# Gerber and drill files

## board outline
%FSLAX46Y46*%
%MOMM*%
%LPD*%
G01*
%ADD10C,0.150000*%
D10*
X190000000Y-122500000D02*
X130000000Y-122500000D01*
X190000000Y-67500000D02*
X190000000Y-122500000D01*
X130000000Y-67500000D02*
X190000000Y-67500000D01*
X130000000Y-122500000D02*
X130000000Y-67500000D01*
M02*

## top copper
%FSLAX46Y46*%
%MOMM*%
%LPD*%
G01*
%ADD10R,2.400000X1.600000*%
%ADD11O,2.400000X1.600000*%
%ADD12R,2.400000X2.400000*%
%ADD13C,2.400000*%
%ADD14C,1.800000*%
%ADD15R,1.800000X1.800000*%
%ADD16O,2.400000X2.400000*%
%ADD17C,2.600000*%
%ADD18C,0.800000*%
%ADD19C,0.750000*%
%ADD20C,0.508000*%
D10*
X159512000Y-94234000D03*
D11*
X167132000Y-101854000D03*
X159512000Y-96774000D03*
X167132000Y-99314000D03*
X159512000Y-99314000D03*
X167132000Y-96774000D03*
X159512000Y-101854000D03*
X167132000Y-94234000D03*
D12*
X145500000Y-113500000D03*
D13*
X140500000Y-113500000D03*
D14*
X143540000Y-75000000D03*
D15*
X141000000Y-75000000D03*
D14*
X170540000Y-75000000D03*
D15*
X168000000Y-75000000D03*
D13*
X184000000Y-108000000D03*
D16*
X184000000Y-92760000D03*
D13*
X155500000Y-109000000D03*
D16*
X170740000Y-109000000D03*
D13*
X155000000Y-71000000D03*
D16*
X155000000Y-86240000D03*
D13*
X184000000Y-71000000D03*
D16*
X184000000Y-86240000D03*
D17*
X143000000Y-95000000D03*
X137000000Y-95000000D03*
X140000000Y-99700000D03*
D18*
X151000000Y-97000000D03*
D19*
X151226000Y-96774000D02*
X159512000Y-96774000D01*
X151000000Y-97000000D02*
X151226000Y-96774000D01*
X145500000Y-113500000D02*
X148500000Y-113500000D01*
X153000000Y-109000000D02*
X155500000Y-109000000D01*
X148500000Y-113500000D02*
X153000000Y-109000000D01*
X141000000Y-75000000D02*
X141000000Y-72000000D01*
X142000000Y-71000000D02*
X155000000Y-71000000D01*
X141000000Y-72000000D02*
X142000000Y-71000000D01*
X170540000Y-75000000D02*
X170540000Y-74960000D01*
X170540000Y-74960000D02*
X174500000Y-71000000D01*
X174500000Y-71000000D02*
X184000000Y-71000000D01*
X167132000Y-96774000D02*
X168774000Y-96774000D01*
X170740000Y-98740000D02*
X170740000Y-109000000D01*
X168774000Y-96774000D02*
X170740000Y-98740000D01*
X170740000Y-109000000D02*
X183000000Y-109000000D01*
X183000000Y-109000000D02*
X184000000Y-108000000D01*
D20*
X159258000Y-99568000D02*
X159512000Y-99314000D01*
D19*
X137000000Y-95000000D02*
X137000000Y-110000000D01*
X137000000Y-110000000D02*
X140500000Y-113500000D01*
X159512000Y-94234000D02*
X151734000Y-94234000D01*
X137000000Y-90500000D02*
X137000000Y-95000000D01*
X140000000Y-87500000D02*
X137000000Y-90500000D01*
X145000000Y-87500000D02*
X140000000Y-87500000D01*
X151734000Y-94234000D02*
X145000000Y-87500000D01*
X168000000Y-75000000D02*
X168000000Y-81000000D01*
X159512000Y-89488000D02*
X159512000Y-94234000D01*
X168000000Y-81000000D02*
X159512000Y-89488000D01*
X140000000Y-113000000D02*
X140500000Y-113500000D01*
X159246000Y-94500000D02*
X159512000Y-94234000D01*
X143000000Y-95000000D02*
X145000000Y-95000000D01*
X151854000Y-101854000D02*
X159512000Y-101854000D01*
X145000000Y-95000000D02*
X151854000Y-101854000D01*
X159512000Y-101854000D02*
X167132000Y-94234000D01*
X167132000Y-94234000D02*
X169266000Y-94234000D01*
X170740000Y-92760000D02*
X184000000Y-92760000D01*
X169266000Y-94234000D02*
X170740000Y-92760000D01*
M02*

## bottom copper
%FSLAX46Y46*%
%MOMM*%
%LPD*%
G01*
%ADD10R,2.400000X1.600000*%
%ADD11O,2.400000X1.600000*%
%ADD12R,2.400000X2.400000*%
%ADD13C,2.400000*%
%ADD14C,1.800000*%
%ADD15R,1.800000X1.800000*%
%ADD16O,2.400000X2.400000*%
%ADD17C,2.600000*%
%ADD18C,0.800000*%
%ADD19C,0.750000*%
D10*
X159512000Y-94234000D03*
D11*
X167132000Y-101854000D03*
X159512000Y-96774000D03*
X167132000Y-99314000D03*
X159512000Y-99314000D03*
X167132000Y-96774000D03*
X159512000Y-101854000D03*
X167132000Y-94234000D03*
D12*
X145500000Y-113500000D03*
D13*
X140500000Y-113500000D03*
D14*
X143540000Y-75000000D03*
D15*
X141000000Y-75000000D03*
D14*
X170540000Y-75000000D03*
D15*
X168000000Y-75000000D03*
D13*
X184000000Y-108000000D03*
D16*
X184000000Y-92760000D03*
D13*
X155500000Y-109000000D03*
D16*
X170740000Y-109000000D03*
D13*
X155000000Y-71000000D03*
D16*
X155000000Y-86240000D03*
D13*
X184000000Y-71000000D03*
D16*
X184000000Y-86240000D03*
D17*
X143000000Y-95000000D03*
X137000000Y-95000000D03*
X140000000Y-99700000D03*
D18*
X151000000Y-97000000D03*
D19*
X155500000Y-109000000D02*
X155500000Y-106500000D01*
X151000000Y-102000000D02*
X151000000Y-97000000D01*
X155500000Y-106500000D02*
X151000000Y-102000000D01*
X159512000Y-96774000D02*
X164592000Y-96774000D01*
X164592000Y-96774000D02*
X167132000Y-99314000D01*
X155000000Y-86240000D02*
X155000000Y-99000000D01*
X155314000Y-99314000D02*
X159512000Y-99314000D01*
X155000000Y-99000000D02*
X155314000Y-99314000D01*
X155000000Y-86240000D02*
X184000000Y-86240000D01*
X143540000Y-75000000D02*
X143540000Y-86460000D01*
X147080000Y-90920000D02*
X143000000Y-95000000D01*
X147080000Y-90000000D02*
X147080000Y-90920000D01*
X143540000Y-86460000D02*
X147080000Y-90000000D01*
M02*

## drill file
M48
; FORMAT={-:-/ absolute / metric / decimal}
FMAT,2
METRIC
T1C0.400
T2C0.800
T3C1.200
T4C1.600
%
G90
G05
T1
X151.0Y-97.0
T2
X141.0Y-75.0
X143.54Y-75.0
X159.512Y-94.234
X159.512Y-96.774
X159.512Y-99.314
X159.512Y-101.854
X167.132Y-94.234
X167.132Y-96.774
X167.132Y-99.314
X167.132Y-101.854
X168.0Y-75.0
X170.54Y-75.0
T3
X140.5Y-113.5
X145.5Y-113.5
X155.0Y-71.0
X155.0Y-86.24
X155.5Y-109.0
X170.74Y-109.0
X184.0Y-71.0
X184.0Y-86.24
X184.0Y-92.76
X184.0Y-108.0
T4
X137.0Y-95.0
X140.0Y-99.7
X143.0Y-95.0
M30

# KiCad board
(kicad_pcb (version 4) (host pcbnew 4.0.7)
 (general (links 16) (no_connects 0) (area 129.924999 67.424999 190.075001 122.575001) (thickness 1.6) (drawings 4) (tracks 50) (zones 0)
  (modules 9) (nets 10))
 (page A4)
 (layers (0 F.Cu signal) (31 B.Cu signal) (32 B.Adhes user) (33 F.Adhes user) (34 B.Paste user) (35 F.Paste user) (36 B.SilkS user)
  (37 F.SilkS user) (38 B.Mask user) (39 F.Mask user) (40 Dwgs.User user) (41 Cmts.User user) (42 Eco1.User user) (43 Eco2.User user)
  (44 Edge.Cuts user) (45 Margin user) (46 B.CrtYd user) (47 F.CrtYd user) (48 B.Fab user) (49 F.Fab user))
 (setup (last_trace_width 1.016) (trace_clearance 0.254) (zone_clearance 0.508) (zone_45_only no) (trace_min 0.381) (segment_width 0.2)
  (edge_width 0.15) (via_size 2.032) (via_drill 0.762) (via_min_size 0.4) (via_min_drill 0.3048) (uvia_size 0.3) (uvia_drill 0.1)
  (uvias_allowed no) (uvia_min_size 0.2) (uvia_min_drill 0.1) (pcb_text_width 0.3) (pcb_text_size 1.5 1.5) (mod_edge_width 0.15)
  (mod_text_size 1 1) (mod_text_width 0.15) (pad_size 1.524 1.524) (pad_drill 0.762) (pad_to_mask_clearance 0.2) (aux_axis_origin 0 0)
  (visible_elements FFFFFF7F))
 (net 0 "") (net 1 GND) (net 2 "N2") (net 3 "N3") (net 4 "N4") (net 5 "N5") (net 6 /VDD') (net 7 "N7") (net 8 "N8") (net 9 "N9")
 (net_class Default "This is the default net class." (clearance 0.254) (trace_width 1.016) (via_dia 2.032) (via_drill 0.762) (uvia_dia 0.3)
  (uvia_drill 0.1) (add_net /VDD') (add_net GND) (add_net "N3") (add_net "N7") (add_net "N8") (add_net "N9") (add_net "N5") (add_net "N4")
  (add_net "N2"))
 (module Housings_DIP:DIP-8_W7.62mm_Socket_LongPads (layer F.Cu) (at 159.512 94.234)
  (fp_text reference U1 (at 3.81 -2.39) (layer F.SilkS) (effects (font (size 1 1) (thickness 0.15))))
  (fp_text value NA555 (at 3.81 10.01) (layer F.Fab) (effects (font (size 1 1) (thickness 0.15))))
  (pad 1 thru_hole rect (at 0 0) (size 2.4 1.6) (drill 0.8) (layers *.Cu *.Mask) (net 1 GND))
  (pad 5 thru_hole oval (at 7.62 7.62) (size 2.4 1.6) (drill 0.8) (layers *.Cu *.Mask) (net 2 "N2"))
  (pad 2 thru_hole oval (at 0 2.54) (size 2.4 1.6) (drill 0.8) (layers *.Cu *.Mask) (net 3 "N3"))
  (pad 6 thru_hole oval (at 7.62 5.08) (size 2.4 1.6) (drill 0.8) (layers *.Cu *.Mask) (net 3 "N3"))
  (pad 3 thru_hole oval (at 0 5.08) (size 2.4 1.6) (drill 0.8) (layers *.Cu *.Mask) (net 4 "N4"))
  (pad 7 thru_hole oval (at 7.62 2.54) (size 2.4 1.6) (drill 0.8) (layers *.Cu *.Mask) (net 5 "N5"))
  (pad 4 thru_hole oval (at 0 7.62) (size 2.4 1.6) (drill 0.8) (layers *.Cu *.Mask) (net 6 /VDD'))
  (pad 8 thru_hole oval (at 7.62 0) (size 2.4 1.6) (drill 0.8) (layers *.Cu *.Mask) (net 6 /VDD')))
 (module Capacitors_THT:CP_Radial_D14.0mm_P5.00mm (layer F.Cu) (at 145.5 113.5 180)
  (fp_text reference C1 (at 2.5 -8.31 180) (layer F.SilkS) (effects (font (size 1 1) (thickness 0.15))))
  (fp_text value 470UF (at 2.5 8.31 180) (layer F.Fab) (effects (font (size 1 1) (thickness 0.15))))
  (pad 1 thru_hole rect (at 0 0 180) (size 2.4 2.4) (drill 1.2) (layers *.Cu *.Mask) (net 3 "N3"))
  (pad 2 thru_hole circle (at 5 0 180) (size 2.4 2.4) (drill 1.2) (layers *.Cu *.Mask) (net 1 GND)))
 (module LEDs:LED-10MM (layer F.Cu) (at 141 75)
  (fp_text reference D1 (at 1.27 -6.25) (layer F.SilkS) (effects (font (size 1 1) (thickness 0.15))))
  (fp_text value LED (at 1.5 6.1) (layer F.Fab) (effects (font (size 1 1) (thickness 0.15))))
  (pad 2 thru_hole circle (at 2.54 0 180) (size 1.8 1.8) (drill 0.8) (layers *.Cu *.Mask) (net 6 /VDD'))
  (pad 1 thru_hole rect (at 0 0 180) (size 1.8 1.8) (drill 0.8) (layers *.Cu *.Mask) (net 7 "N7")))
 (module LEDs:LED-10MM (layer F.Cu) (at 168 75)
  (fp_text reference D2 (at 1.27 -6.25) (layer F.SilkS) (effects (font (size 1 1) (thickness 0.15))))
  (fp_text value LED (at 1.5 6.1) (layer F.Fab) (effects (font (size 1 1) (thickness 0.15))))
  (pad 2 thru_hole circle (at 2.54 0 180) (size 1.8 1.8) (drill 0.8) (layers *.Cu *.Mask) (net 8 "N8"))
  (pad 1 thru_hole rect (at 0 0 180) (size 1.8 1.8) (drill 0.8) (layers *.Cu *.Mask) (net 1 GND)))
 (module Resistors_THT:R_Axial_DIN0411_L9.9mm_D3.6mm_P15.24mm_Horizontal (layer F.Cu) (at 184 108 90)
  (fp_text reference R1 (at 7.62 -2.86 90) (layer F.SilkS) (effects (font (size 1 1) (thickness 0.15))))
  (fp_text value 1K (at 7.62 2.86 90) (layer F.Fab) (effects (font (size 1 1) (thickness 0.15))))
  (pad 1 thru_hole circle (at 0 0 90) (size 2.4 2.4) (drill 1.2) (layers *.Cu *.Mask) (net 5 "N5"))
  (pad 2 thru_hole oval (at 15.24 0 90) (size 2.4 2.4) (drill 1.2) (layers *.Cu *.Mask) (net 6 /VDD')))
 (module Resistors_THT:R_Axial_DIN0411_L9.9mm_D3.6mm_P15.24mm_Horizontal (layer F.Cu) (at 155.5 109)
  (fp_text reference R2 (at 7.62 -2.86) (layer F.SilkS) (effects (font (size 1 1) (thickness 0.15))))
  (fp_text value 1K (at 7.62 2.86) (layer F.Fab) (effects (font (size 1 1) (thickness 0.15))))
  (pad 1 thru_hole circle (at 0 0) (size 2.4 2.4) (drill 1.2) (layers *.Cu *.Mask) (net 3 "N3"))
  (pad 2 thru_hole oval (at 15.24 0) (size 2.4 2.4) (drill 1.2) (layers *.Cu *.Mask) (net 5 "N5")))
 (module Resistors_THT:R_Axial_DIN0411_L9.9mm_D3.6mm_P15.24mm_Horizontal (layer F.Cu) (at 155 71 270)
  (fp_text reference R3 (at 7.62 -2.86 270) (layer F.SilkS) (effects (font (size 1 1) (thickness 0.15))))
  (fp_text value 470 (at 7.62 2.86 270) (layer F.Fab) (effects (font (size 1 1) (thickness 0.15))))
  (pad 1 thru_hole circle (at 0 0 270) (size 2.4 2.4) (drill 1.2) (layers *.Cu *.Mask) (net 7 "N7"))
  (pad 2 thru_hole oval (at 15.24 0 270) (size 2.4 2.4) (drill 1.2) (layers *.Cu *.Mask) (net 4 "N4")))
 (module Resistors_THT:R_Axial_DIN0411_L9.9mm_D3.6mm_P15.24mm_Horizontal (layer F.Cu) (at 184 71 270)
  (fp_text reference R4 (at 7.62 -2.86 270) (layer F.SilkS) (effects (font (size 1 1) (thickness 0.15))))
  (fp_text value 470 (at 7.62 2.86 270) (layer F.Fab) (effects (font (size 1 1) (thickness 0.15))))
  (pad 1 thru_hole circle (at 0 0 270) (size 2.4 2.4) (drill 1.2) (layers *.Cu *.Mask) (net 8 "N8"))
  (pad 2 thru_hole oval (at 15.24 0 270) (size 2.4 2.4) (drill 1.2) (layers *.Cu *.Mask) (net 4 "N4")))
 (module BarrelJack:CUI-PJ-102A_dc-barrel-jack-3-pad (layer F.Cu) (at 140 95 90)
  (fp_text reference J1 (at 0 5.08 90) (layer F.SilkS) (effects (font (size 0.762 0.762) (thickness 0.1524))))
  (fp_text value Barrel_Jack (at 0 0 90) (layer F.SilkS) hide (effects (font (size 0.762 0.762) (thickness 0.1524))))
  (pad 1 thru_hole circle (at 0 3 90) (size 2.6 2.6) (drill 1.6) (layers *.Cu *.Mask F.SilkS) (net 6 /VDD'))
  (pad 2 thru_hole circle (at 0 -3 90) (size 2.6 2.6) (drill 1.6) (layers *.Cu *.Mask F.SilkS) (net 1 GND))
  (pad 3 thru_hole circle (at -4.7 0 90) (size 2.6 2.6) (drill 1.6) (layers *.Cu *.Mask F.SilkS) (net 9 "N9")))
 (gr_line (start 190 122.5) (end 130 122.5) (angle 90) (layer Edge.Cuts) (width 0.15))
 (gr_line (start 190 67.5) (end 190 122.5) (angle 90) (layer Edge.Cuts) (width 0.15))
 (gr_line (start 130 67.5) (end 190 67.5) (angle 90) (layer Edge.Cuts) (width 0.15))
 (gr_line (start 130 122.5) (end 130 67.5) (angle 90) (layer Edge.Cuts) (width 0.15))
 (segment (start 155.5 109) (end 155.5 106.5) (width 0.75) (layer B.Cu) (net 3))
 (segment (start 151.226 96.774) (end 159.512 96.774) (width 0.75) (layer F.Cu) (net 3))
 (segment (start 151 97) (end 151.226 96.774) (width 0.75) (layer F.Cu) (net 3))
 (via (at 151 97) (size 0.8) (drill 0.4) (layers F.Cu B.Cu) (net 3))
 (segment (start 151 102) (end 151 97) (width 0.75) (layer B.Cu) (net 3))
 (segment (start 155.5 106.5) (end 151 102) (width 0.75) (layer B.Cu) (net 3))
 (segment (start 159.512 96.774) (end 164.592 96.774) (width 0.75) (layer B.Cu) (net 3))
 (segment (start 164.592 96.774) (end 167.132 99.314) (width 0.75) (layer B.Cu) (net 3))
 (segment (start 145.5 113.5) (end 148.5 113.5) (width 0.75) (layer F.Cu) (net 3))
 (segment (start 153 109) (end 155.5 109) (width 0.75) (layer F.Cu) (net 3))
 (segment (start 148.5 113.5) (end 153 109) (width 0.75) (layer F.Cu) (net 3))
 (segment (start 141 75) (end 141 72) (width 0.75) (layer F.Cu) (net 7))
 (segment (start 142 71) (end 155 71) (width 0.75) (layer F.Cu) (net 7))
 (segment (start 141 72) (end 142 71) (width 0.75) (layer F.Cu) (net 7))
 (segment (start 170.54 75) (end 170.54 74.96) (width 0.75) (layer F.Cu) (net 8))
 (segment (start 170.54 74.96) (end 174.5 71) (width 0.75) (layer F.Cu) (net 8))
 (segment (start 174.5 71) (end 184 71) (width 0.75) (layer F.Cu) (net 8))
 (segment (start 167.132 96.774) (end 168.774 96.774) (width 0.75) (layer F.Cu) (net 5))
 (segment (start 170.74 98.74) (end 170.74 109) (width 0.75) (layer F.Cu) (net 5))
 (segment (start 168.774 96.774) (end 170.74 98.74) (width 0.75) (layer F.Cu) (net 5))
 (segment (start 170.74 109) (end 183 109) (width 0.75) (layer F.Cu) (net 5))
 (segment (start 183 109) (end 184 108) (width 0.75) (layer F.Cu) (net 5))
 (segment (start 155 86.24) (end 155 99) (width 0.75) (layer B.Cu) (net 4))
 (segment (start 155.314 99.314) (end 159.512 99.314) (width 0.75) (layer B.Cu) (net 4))
 (segment (start 155 99) (end 155.314 99.314) (width 0.75) (layer B.Cu) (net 4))
 (segment (start 155 86.24) (end 184 86.24) (width 0.75) (layer B.Cu) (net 4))
 (segment (start 159.258 99.568) (end 159.512 99.314) (width 0.508) (layer F.Cu) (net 4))
 (segment (start 137 95) (end 137 110) (width 0.75) (layer F.Cu) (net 1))
 (segment (start 137 110) (end 140.5 113.5) (width 0.75) (layer F.Cu) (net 1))
 (segment (start 159.512 94.234) (end 151.734 94.234) (width 0.75) (layer F.Cu) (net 1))
 (segment (start 137 90.5) (end 137 95) (width 0.75) (layer F.Cu) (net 1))
 (segment (start 140 87.5) (end 137 90.5) (width 0.75) (layer F.Cu) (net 1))
 (segment (start 145 87.5) (end 140 87.5) (width 0.75) (layer F.Cu) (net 1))
 (segment (start 151.734 94.234) (end 145 87.5) (width 0.75) (layer F.Cu) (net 1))
 (segment (start 168 75) (end 168 81) (width 0.75) (layer F.Cu) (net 1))
 (segment (start 159.512 89.488) (end 159.512 94.234) (width 0.75) (layer F.Cu) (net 1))
 (segment (start 168 81) (end 159.512 89.488) (width 0.75) (layer F.Cu) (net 1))
 (segment (start 140 113) (end 140.5 113.5) (width 0.75) (layer F.Cu) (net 1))
 (segment (start 159.246 94.5) (end 159.512 94.234) (width 0.75) (layer F.Cu) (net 1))
 (segment (start 143.54 75) (end 143.54 86.46) (width 0.75) (layer B.Cu) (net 6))
 (segment (start 147.08 90.92) (end 143 95) (width 0.75) (layer B.Cu) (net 6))
 (segment (start 147.08 90) (end 147.08 90.92) (width 0.75) (layer B.Cu) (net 6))
 (segment (start 143.54 86.46) (end 147.08 90) (width 0.75) (layer B.Cu) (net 6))
 (segment (start 143 95) (end 145 95) (width 0.75) (layer F.Cu) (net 6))
 (segment (start 151.854 101.854) (end 159.512 101.854) (width 0.75) (layer F.Cu) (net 6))
 (segment (start 145 95) (end 151.854 101.854) (width 0.75) (layer F.Cu) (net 6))
 (segment (start 159.512 101.854) (end 167.132 94.234) (width 0.75) (layer F.Cu) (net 6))
 (segment (start 167.132 94.234) (end 169.266 94.234) (width 0.75) (layer F.Cu) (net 6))
 (segment (start 170.74 92.76) (end 184 92.76) (width 0.75) (layer F.Cu) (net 6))
 (segment (start 169.266 94.234) (end 170.74 92.76) (width 0.75) (layer F.Cu) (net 6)))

